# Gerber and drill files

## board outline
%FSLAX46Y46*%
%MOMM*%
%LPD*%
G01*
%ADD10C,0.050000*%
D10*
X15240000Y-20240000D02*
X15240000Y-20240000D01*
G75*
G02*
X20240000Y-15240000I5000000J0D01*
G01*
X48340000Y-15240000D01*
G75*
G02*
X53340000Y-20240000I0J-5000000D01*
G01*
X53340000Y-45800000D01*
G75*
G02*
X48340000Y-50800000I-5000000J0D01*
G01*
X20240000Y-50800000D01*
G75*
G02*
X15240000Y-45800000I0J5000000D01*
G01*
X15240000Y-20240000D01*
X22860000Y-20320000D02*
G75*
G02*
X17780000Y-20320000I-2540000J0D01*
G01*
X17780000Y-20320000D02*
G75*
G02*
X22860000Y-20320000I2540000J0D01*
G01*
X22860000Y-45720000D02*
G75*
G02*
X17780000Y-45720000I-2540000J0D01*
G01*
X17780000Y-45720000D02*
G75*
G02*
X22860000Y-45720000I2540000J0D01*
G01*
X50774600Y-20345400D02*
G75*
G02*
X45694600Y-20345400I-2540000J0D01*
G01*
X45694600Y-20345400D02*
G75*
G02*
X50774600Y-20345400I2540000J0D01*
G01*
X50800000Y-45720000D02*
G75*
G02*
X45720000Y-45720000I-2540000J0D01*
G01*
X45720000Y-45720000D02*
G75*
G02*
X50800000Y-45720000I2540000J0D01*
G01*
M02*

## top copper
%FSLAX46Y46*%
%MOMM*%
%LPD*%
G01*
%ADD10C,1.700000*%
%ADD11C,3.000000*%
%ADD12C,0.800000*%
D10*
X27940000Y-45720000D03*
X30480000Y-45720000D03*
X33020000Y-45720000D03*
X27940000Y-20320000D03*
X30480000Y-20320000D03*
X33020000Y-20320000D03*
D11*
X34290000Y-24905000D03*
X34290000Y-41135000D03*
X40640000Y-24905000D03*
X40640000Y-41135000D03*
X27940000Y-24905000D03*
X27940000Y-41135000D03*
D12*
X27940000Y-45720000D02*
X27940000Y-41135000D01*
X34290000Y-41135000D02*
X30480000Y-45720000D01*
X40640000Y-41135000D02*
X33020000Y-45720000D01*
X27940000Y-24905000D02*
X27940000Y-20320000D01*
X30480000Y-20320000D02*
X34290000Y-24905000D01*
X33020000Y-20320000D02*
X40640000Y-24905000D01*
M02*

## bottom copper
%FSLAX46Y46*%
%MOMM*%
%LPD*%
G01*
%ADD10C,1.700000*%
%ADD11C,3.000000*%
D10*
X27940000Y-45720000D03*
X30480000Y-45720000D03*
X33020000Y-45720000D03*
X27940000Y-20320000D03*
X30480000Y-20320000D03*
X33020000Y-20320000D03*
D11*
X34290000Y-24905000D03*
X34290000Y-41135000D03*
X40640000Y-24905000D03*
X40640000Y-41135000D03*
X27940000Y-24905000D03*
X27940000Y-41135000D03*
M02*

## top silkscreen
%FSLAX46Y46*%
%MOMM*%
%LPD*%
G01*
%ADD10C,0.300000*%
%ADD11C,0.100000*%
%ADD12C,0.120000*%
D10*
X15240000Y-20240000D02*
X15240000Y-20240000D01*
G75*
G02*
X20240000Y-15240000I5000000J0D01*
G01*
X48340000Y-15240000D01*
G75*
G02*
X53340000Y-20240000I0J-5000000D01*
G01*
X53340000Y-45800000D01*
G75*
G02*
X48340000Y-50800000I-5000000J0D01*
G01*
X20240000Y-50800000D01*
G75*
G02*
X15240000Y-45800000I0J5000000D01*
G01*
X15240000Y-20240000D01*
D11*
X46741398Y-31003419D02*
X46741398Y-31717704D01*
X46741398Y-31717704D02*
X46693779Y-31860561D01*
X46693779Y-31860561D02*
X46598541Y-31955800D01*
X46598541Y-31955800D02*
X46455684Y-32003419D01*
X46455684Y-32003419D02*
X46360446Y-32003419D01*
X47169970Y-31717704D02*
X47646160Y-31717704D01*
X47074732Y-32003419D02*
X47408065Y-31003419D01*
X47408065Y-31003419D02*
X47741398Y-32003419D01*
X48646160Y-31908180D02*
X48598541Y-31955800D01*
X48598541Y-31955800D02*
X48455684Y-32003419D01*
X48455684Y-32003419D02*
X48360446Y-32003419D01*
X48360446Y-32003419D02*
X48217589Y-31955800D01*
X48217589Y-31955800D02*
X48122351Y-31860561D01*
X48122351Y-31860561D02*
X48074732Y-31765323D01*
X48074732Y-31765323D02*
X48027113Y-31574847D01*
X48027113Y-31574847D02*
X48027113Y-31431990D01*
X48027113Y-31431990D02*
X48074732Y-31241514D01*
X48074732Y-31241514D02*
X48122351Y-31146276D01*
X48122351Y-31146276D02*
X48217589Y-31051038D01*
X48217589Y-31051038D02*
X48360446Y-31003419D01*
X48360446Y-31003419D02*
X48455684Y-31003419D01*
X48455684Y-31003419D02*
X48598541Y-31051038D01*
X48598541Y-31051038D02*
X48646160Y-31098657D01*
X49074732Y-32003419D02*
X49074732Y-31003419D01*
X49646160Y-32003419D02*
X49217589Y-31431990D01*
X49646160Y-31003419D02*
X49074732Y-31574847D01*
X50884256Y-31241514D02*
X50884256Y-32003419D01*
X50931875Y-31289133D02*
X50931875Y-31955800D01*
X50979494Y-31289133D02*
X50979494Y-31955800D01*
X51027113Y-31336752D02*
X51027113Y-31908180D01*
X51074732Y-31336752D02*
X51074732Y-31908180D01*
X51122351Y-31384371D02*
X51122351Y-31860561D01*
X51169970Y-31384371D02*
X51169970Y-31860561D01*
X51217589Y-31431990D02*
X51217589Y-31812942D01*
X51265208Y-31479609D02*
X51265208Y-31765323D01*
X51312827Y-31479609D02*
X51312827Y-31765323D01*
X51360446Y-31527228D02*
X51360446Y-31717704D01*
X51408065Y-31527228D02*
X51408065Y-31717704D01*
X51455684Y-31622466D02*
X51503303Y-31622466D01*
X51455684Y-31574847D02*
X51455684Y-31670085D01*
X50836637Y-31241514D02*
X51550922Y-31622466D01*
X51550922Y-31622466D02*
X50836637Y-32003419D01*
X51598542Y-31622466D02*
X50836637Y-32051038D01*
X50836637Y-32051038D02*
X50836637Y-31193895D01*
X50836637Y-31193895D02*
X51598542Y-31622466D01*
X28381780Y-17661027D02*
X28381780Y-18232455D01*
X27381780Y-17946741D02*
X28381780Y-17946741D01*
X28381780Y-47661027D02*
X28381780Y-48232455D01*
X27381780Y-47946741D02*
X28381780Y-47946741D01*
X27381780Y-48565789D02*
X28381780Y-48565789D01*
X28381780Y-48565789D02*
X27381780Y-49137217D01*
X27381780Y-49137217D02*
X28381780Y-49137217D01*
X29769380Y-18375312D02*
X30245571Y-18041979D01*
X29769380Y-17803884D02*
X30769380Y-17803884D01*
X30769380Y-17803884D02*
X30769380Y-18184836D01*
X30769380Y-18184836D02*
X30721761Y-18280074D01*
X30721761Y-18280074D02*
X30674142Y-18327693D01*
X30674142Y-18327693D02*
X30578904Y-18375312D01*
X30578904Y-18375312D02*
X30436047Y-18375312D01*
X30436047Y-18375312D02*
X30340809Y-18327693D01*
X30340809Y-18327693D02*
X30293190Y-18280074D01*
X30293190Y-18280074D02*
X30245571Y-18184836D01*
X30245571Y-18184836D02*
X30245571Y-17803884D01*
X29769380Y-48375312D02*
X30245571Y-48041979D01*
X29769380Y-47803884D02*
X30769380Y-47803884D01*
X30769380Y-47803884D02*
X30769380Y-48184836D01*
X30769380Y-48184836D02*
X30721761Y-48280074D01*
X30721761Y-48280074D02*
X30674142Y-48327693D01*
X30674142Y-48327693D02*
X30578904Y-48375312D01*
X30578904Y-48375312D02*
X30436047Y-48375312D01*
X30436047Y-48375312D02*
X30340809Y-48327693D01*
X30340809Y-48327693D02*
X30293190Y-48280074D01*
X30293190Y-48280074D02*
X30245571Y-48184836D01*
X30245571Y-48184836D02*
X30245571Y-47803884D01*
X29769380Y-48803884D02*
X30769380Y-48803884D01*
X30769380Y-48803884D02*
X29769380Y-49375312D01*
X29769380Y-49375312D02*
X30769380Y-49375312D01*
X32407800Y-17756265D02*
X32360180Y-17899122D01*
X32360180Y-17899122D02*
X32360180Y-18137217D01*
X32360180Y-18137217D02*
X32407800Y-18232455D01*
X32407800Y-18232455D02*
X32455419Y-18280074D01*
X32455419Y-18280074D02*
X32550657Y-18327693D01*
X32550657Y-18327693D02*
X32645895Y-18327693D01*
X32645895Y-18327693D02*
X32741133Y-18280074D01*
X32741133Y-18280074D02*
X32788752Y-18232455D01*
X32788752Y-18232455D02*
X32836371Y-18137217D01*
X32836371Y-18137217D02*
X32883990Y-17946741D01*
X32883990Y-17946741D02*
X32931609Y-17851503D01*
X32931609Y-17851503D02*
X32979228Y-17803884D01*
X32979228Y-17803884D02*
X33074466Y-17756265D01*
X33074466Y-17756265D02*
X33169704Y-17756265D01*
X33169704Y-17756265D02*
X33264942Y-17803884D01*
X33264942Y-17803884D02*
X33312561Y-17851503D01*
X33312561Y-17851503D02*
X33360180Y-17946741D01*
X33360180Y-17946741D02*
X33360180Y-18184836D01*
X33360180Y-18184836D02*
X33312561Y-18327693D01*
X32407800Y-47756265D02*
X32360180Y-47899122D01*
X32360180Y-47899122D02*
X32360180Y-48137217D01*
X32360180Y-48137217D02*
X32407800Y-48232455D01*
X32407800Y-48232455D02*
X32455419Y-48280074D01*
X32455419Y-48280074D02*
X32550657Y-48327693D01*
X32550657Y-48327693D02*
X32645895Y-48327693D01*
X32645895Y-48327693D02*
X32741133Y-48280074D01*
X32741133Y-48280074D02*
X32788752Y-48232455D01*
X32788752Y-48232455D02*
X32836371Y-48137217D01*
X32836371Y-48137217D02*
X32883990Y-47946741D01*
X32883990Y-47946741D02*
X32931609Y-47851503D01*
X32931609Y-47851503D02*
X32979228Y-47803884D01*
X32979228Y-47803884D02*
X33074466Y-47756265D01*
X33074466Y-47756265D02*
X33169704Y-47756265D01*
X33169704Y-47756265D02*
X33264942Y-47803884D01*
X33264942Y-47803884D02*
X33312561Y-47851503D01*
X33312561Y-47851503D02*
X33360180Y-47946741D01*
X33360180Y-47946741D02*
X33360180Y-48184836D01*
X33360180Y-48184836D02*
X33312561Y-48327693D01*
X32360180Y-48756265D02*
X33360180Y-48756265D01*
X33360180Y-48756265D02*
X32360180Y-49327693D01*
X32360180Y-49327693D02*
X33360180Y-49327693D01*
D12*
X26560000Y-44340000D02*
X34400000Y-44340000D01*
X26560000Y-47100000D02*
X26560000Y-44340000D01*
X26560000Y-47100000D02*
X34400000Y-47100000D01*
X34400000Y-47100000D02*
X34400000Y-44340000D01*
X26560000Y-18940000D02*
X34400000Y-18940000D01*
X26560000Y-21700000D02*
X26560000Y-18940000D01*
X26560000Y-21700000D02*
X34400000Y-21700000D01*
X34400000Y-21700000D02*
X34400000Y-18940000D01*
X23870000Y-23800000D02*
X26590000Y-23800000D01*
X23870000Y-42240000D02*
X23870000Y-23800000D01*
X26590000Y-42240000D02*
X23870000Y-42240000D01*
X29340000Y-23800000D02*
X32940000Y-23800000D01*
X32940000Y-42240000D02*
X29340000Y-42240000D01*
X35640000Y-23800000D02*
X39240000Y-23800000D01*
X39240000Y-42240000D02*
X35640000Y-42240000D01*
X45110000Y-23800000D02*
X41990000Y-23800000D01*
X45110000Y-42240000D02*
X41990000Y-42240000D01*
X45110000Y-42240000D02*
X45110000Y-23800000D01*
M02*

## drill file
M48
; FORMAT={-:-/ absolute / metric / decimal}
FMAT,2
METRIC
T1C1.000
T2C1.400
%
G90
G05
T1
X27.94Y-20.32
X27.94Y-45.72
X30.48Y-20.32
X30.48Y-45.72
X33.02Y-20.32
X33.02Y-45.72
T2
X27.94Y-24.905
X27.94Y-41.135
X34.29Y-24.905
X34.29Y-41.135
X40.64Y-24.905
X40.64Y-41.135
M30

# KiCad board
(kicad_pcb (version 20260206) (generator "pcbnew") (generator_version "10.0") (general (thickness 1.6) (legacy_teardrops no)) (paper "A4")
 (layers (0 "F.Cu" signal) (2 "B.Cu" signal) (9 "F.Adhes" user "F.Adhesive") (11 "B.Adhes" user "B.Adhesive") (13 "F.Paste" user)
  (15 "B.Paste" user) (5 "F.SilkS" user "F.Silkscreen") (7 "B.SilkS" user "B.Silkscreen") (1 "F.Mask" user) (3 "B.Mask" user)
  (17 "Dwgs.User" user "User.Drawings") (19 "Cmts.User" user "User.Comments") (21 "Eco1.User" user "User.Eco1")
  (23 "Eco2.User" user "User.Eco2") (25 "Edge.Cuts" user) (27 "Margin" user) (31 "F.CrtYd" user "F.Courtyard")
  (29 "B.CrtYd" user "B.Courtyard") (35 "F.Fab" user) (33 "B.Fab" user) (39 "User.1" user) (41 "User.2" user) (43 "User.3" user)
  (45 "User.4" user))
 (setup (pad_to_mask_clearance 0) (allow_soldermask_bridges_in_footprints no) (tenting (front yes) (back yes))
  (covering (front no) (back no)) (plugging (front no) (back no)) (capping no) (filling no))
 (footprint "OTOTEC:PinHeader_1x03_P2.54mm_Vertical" (layer "F.Cu") (at 27.94 45.72 90)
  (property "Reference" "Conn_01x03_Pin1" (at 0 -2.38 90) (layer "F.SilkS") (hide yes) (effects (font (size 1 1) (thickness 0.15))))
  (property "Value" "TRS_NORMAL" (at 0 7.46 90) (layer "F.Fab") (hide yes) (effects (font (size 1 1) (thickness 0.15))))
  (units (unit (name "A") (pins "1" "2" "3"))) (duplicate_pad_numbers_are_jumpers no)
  (fp_line (start 1.38 -1.38) (end 1.38 6.46) (stroke (width 0.12) (type solid)) (layer "F.SilkS"))
  (fp_line (start -1.38 -1.38) (end 1.38 -1.38) (stroke (width 0.12) (type solid)) (layer "F.SilkS"))
  (fp_line (start -1.38 -1.38) (end -1.38 6.46) (stroke (width 0.12) (type solid)) (layer "F.SilkS"))
  (fp_line (start -1.38 6.46) (end 1.38 6.46) (stroke (width 0.12) (type solid)) (layer "F.SilkS"))
  (pad "1" thru_hole circle (at 0 0 90) (size 1.7 1.7) (drill 1) (layers "*.Cu" "*.Mask") (remove_unused_layers no)
   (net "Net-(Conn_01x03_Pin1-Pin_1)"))
  (pad "2" thru_hole circle (at 0 2.54 90) (size 1.7 1.7) (drill 1) (layers "*.Cu" "*.Mask") (remove_unused_layers no)
   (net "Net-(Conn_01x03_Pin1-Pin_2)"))
  (pad "3" thru_hole circle (at 0 5.08 90) (size 1.7 1.7) (drill 1) (layers "*.Cu" "*.Mask") (remove_unused_layers no)
   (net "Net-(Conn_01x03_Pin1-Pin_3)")))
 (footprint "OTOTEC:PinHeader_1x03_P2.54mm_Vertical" (layer "F.Cu") (at 27.94 20.32 90)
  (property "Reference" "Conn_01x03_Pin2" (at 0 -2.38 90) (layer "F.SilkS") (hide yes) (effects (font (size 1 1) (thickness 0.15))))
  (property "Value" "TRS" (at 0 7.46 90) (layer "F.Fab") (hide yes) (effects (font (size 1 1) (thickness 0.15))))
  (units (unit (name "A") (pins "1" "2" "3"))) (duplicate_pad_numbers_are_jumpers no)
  (fp_line (start 1.38 -1.38) (end 1.38 6.46) (stroke (width 0.12) (type solid)) (layer "F.SilkS"))
  (fp_line (start -1.38 -1.38) (end 1.38 -1.38) (stroke (width 0.12) (type solid)) (layer "F.SilkS"))
  (fp_line (start -1.38 -1.38) (end -1.38 6.46) (stroke (width 0.12) (type solid)) (layer "F.SilkS"))
  (fp_line (start -1.38 6.46) (end 1.38 6.46) (stroke (width 0.12) (type solid)) (layer "F.SilkS"))
  (pad "1" thru_hole circle (at 0 0 90) (size 1.7 1.7) (drill 1) (layers "*.Cu" "*.Mask") (remove_unused_layers no)
   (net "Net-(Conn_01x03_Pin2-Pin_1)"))
  (pad "2" thru_hole circle (at 0 2.54 90) (size 1.7 1.7) (drill 1) (layers "*.Cu" "*.Mask") (remove_unused_layers no)
   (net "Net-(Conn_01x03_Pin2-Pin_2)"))
  (pad "3" thru_hole circle (at 0 5.08 90) (size 1.7 1.7) (drill 1) (layers "*.Cu" "*.Mask") (remove_unused_layers no)
   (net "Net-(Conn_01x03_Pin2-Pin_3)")))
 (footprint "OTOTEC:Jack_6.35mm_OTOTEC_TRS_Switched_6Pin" (layer "F.Cu") (at 27.94 24.905)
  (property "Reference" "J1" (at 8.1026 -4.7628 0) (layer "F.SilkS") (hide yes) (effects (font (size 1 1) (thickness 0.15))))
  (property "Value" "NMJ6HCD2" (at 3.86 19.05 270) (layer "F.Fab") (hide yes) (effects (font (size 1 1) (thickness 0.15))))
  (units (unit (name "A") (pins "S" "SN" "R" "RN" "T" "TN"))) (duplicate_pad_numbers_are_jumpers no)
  (fp_line (start -4.07 -1.105) (end -1.35 -1.105) (stroke (width 0.12) (type solid)) (layer "F.SilkS"))
  (fp_line (start -4.07 17.335) (end -4.07 -1.105) (stroke (width 0.12) (type solid)) (layer "F.SilkS"))
  (fp_line (start -1.35 17.335) (end -4.07 17.335) (stroke (width 0.12) (type solid)) (layer "F.SilkS"))
  (fp_line (start 1.4 -1.105) (end 5 -1.105) (stroke (width 0.12) (type solid)) (layer "F.SilkS"))
  (fp_line (start 5 17.335) (end 1.4 17.335) (stroke (width 0.12) (type solid)) (layer "F.SilkS"))
  (fp_line (start 7.7 -1.105) (end 11.3 -1.105) (stroke (width 0.12) (type solid)) (layer "F.SilkS"))
  (fp_line (start 11.3 17.335) (end 7.7 17.335) (stroke (width 0.12) (type solid)) (layer "F.SilkS"))
  (fp_line (start 17.17 -1.105) (end 14.05 -1.105) (stroke (width 0.12) (type solid)) (layer "F.SilkS"))
  (fp_line (start 17.17 17.335) (end 14.05 17.335) (stroke (width 0.12) (type solid)) (layer "F.SilkS"))
  (fp_line (start 17.17 17.335) (end 17.17 -1.105) (stroke (width 0.12) (type solid)) (layer "F.SilkS"))
  (pad "R" thru_hole circle (at 6.35 0) (size 3 3) (drill 1.4) (layers "*.Cu" "*.Mask") (remove_unused_layers no)
   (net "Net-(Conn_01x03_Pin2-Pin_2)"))
  (pad "RN" thru_hole circle (at 6.35 16.23) (size 3 3) (drill 1.4) (layers "*.Cu" "*.Mask") (remove_unused_layers no)
   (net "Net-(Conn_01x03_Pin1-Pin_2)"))
  (pad "S" thru_hole circle (at 12.7 0) (size 3 3) (drill 1.4) (layers "*.Cu" "*.Mask") (remove_unused_layers no)
   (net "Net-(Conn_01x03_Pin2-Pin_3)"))
  (pad "SN" thru_hole circle (at 12.7 16.23) (size 3 3) (drill 1.4) (layers "*.Cu" "*.Mask") (remove_unused_layers no)
   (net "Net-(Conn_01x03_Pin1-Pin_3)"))
  (pad "T" thru_hole circle (at 0 0) (size 3 3) (drill 1.4) (layers "*.Cu" "*.Mask") (remove_unused_layers no)
   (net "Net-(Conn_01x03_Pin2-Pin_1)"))
  (pad "TN" thru_hole circle (at 0 16.23) (size 3 3) (drill 1.4) (layers "*.Cu" "*.Mask") (remove_unused_layers no)
   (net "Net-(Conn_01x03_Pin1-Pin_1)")))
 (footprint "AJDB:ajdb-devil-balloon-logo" (layer "B.Cu") (at 34.3154 32.9946 90)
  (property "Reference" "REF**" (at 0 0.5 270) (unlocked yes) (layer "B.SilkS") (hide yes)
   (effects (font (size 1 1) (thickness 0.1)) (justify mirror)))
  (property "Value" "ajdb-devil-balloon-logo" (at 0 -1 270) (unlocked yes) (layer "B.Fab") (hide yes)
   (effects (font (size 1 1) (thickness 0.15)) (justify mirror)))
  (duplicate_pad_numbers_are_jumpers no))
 (gr_rect (start 15.24 15.24) (end 53.34 50.8) (radius 5) (stroke (width 0.3) (type solid)) (fill no) (layer "F.SilkS"))
 (gr_rect (start 15.24 15.24) (end 53.34 50.8) (radius 5) (stroke (width 0.05) (type solid)) (fill no) (layer "Edge.Cuts"))
 (gr_circle (center 20.32 20.32) (end 17.78 20.32) (stroke (width 0.05) (type default)) (fill no) (locked yes) (layer "Edge.Cuts"))
 (gr_circle (center 20.32 45.72) (end 22.86 45.72) (stroke (width 0.05) (type solid)) (fill no) (locked yes) (layer "Edge.Cuts"))
 (gr_circle (center 48.2346 20.3454) (end 48.2346 22.8854) (stroke (width 0.05) (type default)) (fill no) (locked yes) (layer "Edge.Cuts"))
 (gr_circle (center 48.26 45.72) (end 48.26 48.26) (stroke (width 0.05) (type default)) (fill no) (locked yes) (layer "Edge.Cuts"))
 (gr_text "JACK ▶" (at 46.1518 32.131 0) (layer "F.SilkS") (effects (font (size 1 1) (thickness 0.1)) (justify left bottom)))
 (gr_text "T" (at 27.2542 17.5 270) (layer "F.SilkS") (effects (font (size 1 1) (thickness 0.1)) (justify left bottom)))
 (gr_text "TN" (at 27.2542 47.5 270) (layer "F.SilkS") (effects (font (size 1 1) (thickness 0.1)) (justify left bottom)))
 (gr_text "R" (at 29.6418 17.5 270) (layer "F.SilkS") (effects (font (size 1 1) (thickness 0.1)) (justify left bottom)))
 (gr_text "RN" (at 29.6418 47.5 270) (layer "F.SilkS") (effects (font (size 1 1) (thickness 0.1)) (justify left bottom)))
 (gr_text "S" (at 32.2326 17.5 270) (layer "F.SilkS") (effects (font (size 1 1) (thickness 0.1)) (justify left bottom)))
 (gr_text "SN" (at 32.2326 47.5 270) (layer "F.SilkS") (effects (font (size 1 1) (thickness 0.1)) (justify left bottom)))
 (segment (start 27.94 45.72) (end 27.94 41.135) (width 0.8) (layer "F.Cu") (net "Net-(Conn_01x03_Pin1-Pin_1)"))
 (segment (start 34.29 41.135) (end 30.48 45.72) (width 0.8) (layer "F.Cu") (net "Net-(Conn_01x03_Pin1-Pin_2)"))
 (segment (start 40.64 41.135) (end 33.02 45.72) (width 0.8) (layer "F.Cu") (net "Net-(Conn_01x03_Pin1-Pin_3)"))
 (segment (start 27.94 24.905) (end 27.94 20.32) (width 0.8) (layer "F.Cu") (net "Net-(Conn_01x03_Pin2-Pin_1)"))
 (segment (start 30.48 20.32) (end 34.29 24.905) (width 0.8) (layer "F.Cu") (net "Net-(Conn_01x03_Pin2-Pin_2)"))
 (segment (start 33.02 20.32) (end 40.64 24.905) (width 0.8) (layer "F.Cu") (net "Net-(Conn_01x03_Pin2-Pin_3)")))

